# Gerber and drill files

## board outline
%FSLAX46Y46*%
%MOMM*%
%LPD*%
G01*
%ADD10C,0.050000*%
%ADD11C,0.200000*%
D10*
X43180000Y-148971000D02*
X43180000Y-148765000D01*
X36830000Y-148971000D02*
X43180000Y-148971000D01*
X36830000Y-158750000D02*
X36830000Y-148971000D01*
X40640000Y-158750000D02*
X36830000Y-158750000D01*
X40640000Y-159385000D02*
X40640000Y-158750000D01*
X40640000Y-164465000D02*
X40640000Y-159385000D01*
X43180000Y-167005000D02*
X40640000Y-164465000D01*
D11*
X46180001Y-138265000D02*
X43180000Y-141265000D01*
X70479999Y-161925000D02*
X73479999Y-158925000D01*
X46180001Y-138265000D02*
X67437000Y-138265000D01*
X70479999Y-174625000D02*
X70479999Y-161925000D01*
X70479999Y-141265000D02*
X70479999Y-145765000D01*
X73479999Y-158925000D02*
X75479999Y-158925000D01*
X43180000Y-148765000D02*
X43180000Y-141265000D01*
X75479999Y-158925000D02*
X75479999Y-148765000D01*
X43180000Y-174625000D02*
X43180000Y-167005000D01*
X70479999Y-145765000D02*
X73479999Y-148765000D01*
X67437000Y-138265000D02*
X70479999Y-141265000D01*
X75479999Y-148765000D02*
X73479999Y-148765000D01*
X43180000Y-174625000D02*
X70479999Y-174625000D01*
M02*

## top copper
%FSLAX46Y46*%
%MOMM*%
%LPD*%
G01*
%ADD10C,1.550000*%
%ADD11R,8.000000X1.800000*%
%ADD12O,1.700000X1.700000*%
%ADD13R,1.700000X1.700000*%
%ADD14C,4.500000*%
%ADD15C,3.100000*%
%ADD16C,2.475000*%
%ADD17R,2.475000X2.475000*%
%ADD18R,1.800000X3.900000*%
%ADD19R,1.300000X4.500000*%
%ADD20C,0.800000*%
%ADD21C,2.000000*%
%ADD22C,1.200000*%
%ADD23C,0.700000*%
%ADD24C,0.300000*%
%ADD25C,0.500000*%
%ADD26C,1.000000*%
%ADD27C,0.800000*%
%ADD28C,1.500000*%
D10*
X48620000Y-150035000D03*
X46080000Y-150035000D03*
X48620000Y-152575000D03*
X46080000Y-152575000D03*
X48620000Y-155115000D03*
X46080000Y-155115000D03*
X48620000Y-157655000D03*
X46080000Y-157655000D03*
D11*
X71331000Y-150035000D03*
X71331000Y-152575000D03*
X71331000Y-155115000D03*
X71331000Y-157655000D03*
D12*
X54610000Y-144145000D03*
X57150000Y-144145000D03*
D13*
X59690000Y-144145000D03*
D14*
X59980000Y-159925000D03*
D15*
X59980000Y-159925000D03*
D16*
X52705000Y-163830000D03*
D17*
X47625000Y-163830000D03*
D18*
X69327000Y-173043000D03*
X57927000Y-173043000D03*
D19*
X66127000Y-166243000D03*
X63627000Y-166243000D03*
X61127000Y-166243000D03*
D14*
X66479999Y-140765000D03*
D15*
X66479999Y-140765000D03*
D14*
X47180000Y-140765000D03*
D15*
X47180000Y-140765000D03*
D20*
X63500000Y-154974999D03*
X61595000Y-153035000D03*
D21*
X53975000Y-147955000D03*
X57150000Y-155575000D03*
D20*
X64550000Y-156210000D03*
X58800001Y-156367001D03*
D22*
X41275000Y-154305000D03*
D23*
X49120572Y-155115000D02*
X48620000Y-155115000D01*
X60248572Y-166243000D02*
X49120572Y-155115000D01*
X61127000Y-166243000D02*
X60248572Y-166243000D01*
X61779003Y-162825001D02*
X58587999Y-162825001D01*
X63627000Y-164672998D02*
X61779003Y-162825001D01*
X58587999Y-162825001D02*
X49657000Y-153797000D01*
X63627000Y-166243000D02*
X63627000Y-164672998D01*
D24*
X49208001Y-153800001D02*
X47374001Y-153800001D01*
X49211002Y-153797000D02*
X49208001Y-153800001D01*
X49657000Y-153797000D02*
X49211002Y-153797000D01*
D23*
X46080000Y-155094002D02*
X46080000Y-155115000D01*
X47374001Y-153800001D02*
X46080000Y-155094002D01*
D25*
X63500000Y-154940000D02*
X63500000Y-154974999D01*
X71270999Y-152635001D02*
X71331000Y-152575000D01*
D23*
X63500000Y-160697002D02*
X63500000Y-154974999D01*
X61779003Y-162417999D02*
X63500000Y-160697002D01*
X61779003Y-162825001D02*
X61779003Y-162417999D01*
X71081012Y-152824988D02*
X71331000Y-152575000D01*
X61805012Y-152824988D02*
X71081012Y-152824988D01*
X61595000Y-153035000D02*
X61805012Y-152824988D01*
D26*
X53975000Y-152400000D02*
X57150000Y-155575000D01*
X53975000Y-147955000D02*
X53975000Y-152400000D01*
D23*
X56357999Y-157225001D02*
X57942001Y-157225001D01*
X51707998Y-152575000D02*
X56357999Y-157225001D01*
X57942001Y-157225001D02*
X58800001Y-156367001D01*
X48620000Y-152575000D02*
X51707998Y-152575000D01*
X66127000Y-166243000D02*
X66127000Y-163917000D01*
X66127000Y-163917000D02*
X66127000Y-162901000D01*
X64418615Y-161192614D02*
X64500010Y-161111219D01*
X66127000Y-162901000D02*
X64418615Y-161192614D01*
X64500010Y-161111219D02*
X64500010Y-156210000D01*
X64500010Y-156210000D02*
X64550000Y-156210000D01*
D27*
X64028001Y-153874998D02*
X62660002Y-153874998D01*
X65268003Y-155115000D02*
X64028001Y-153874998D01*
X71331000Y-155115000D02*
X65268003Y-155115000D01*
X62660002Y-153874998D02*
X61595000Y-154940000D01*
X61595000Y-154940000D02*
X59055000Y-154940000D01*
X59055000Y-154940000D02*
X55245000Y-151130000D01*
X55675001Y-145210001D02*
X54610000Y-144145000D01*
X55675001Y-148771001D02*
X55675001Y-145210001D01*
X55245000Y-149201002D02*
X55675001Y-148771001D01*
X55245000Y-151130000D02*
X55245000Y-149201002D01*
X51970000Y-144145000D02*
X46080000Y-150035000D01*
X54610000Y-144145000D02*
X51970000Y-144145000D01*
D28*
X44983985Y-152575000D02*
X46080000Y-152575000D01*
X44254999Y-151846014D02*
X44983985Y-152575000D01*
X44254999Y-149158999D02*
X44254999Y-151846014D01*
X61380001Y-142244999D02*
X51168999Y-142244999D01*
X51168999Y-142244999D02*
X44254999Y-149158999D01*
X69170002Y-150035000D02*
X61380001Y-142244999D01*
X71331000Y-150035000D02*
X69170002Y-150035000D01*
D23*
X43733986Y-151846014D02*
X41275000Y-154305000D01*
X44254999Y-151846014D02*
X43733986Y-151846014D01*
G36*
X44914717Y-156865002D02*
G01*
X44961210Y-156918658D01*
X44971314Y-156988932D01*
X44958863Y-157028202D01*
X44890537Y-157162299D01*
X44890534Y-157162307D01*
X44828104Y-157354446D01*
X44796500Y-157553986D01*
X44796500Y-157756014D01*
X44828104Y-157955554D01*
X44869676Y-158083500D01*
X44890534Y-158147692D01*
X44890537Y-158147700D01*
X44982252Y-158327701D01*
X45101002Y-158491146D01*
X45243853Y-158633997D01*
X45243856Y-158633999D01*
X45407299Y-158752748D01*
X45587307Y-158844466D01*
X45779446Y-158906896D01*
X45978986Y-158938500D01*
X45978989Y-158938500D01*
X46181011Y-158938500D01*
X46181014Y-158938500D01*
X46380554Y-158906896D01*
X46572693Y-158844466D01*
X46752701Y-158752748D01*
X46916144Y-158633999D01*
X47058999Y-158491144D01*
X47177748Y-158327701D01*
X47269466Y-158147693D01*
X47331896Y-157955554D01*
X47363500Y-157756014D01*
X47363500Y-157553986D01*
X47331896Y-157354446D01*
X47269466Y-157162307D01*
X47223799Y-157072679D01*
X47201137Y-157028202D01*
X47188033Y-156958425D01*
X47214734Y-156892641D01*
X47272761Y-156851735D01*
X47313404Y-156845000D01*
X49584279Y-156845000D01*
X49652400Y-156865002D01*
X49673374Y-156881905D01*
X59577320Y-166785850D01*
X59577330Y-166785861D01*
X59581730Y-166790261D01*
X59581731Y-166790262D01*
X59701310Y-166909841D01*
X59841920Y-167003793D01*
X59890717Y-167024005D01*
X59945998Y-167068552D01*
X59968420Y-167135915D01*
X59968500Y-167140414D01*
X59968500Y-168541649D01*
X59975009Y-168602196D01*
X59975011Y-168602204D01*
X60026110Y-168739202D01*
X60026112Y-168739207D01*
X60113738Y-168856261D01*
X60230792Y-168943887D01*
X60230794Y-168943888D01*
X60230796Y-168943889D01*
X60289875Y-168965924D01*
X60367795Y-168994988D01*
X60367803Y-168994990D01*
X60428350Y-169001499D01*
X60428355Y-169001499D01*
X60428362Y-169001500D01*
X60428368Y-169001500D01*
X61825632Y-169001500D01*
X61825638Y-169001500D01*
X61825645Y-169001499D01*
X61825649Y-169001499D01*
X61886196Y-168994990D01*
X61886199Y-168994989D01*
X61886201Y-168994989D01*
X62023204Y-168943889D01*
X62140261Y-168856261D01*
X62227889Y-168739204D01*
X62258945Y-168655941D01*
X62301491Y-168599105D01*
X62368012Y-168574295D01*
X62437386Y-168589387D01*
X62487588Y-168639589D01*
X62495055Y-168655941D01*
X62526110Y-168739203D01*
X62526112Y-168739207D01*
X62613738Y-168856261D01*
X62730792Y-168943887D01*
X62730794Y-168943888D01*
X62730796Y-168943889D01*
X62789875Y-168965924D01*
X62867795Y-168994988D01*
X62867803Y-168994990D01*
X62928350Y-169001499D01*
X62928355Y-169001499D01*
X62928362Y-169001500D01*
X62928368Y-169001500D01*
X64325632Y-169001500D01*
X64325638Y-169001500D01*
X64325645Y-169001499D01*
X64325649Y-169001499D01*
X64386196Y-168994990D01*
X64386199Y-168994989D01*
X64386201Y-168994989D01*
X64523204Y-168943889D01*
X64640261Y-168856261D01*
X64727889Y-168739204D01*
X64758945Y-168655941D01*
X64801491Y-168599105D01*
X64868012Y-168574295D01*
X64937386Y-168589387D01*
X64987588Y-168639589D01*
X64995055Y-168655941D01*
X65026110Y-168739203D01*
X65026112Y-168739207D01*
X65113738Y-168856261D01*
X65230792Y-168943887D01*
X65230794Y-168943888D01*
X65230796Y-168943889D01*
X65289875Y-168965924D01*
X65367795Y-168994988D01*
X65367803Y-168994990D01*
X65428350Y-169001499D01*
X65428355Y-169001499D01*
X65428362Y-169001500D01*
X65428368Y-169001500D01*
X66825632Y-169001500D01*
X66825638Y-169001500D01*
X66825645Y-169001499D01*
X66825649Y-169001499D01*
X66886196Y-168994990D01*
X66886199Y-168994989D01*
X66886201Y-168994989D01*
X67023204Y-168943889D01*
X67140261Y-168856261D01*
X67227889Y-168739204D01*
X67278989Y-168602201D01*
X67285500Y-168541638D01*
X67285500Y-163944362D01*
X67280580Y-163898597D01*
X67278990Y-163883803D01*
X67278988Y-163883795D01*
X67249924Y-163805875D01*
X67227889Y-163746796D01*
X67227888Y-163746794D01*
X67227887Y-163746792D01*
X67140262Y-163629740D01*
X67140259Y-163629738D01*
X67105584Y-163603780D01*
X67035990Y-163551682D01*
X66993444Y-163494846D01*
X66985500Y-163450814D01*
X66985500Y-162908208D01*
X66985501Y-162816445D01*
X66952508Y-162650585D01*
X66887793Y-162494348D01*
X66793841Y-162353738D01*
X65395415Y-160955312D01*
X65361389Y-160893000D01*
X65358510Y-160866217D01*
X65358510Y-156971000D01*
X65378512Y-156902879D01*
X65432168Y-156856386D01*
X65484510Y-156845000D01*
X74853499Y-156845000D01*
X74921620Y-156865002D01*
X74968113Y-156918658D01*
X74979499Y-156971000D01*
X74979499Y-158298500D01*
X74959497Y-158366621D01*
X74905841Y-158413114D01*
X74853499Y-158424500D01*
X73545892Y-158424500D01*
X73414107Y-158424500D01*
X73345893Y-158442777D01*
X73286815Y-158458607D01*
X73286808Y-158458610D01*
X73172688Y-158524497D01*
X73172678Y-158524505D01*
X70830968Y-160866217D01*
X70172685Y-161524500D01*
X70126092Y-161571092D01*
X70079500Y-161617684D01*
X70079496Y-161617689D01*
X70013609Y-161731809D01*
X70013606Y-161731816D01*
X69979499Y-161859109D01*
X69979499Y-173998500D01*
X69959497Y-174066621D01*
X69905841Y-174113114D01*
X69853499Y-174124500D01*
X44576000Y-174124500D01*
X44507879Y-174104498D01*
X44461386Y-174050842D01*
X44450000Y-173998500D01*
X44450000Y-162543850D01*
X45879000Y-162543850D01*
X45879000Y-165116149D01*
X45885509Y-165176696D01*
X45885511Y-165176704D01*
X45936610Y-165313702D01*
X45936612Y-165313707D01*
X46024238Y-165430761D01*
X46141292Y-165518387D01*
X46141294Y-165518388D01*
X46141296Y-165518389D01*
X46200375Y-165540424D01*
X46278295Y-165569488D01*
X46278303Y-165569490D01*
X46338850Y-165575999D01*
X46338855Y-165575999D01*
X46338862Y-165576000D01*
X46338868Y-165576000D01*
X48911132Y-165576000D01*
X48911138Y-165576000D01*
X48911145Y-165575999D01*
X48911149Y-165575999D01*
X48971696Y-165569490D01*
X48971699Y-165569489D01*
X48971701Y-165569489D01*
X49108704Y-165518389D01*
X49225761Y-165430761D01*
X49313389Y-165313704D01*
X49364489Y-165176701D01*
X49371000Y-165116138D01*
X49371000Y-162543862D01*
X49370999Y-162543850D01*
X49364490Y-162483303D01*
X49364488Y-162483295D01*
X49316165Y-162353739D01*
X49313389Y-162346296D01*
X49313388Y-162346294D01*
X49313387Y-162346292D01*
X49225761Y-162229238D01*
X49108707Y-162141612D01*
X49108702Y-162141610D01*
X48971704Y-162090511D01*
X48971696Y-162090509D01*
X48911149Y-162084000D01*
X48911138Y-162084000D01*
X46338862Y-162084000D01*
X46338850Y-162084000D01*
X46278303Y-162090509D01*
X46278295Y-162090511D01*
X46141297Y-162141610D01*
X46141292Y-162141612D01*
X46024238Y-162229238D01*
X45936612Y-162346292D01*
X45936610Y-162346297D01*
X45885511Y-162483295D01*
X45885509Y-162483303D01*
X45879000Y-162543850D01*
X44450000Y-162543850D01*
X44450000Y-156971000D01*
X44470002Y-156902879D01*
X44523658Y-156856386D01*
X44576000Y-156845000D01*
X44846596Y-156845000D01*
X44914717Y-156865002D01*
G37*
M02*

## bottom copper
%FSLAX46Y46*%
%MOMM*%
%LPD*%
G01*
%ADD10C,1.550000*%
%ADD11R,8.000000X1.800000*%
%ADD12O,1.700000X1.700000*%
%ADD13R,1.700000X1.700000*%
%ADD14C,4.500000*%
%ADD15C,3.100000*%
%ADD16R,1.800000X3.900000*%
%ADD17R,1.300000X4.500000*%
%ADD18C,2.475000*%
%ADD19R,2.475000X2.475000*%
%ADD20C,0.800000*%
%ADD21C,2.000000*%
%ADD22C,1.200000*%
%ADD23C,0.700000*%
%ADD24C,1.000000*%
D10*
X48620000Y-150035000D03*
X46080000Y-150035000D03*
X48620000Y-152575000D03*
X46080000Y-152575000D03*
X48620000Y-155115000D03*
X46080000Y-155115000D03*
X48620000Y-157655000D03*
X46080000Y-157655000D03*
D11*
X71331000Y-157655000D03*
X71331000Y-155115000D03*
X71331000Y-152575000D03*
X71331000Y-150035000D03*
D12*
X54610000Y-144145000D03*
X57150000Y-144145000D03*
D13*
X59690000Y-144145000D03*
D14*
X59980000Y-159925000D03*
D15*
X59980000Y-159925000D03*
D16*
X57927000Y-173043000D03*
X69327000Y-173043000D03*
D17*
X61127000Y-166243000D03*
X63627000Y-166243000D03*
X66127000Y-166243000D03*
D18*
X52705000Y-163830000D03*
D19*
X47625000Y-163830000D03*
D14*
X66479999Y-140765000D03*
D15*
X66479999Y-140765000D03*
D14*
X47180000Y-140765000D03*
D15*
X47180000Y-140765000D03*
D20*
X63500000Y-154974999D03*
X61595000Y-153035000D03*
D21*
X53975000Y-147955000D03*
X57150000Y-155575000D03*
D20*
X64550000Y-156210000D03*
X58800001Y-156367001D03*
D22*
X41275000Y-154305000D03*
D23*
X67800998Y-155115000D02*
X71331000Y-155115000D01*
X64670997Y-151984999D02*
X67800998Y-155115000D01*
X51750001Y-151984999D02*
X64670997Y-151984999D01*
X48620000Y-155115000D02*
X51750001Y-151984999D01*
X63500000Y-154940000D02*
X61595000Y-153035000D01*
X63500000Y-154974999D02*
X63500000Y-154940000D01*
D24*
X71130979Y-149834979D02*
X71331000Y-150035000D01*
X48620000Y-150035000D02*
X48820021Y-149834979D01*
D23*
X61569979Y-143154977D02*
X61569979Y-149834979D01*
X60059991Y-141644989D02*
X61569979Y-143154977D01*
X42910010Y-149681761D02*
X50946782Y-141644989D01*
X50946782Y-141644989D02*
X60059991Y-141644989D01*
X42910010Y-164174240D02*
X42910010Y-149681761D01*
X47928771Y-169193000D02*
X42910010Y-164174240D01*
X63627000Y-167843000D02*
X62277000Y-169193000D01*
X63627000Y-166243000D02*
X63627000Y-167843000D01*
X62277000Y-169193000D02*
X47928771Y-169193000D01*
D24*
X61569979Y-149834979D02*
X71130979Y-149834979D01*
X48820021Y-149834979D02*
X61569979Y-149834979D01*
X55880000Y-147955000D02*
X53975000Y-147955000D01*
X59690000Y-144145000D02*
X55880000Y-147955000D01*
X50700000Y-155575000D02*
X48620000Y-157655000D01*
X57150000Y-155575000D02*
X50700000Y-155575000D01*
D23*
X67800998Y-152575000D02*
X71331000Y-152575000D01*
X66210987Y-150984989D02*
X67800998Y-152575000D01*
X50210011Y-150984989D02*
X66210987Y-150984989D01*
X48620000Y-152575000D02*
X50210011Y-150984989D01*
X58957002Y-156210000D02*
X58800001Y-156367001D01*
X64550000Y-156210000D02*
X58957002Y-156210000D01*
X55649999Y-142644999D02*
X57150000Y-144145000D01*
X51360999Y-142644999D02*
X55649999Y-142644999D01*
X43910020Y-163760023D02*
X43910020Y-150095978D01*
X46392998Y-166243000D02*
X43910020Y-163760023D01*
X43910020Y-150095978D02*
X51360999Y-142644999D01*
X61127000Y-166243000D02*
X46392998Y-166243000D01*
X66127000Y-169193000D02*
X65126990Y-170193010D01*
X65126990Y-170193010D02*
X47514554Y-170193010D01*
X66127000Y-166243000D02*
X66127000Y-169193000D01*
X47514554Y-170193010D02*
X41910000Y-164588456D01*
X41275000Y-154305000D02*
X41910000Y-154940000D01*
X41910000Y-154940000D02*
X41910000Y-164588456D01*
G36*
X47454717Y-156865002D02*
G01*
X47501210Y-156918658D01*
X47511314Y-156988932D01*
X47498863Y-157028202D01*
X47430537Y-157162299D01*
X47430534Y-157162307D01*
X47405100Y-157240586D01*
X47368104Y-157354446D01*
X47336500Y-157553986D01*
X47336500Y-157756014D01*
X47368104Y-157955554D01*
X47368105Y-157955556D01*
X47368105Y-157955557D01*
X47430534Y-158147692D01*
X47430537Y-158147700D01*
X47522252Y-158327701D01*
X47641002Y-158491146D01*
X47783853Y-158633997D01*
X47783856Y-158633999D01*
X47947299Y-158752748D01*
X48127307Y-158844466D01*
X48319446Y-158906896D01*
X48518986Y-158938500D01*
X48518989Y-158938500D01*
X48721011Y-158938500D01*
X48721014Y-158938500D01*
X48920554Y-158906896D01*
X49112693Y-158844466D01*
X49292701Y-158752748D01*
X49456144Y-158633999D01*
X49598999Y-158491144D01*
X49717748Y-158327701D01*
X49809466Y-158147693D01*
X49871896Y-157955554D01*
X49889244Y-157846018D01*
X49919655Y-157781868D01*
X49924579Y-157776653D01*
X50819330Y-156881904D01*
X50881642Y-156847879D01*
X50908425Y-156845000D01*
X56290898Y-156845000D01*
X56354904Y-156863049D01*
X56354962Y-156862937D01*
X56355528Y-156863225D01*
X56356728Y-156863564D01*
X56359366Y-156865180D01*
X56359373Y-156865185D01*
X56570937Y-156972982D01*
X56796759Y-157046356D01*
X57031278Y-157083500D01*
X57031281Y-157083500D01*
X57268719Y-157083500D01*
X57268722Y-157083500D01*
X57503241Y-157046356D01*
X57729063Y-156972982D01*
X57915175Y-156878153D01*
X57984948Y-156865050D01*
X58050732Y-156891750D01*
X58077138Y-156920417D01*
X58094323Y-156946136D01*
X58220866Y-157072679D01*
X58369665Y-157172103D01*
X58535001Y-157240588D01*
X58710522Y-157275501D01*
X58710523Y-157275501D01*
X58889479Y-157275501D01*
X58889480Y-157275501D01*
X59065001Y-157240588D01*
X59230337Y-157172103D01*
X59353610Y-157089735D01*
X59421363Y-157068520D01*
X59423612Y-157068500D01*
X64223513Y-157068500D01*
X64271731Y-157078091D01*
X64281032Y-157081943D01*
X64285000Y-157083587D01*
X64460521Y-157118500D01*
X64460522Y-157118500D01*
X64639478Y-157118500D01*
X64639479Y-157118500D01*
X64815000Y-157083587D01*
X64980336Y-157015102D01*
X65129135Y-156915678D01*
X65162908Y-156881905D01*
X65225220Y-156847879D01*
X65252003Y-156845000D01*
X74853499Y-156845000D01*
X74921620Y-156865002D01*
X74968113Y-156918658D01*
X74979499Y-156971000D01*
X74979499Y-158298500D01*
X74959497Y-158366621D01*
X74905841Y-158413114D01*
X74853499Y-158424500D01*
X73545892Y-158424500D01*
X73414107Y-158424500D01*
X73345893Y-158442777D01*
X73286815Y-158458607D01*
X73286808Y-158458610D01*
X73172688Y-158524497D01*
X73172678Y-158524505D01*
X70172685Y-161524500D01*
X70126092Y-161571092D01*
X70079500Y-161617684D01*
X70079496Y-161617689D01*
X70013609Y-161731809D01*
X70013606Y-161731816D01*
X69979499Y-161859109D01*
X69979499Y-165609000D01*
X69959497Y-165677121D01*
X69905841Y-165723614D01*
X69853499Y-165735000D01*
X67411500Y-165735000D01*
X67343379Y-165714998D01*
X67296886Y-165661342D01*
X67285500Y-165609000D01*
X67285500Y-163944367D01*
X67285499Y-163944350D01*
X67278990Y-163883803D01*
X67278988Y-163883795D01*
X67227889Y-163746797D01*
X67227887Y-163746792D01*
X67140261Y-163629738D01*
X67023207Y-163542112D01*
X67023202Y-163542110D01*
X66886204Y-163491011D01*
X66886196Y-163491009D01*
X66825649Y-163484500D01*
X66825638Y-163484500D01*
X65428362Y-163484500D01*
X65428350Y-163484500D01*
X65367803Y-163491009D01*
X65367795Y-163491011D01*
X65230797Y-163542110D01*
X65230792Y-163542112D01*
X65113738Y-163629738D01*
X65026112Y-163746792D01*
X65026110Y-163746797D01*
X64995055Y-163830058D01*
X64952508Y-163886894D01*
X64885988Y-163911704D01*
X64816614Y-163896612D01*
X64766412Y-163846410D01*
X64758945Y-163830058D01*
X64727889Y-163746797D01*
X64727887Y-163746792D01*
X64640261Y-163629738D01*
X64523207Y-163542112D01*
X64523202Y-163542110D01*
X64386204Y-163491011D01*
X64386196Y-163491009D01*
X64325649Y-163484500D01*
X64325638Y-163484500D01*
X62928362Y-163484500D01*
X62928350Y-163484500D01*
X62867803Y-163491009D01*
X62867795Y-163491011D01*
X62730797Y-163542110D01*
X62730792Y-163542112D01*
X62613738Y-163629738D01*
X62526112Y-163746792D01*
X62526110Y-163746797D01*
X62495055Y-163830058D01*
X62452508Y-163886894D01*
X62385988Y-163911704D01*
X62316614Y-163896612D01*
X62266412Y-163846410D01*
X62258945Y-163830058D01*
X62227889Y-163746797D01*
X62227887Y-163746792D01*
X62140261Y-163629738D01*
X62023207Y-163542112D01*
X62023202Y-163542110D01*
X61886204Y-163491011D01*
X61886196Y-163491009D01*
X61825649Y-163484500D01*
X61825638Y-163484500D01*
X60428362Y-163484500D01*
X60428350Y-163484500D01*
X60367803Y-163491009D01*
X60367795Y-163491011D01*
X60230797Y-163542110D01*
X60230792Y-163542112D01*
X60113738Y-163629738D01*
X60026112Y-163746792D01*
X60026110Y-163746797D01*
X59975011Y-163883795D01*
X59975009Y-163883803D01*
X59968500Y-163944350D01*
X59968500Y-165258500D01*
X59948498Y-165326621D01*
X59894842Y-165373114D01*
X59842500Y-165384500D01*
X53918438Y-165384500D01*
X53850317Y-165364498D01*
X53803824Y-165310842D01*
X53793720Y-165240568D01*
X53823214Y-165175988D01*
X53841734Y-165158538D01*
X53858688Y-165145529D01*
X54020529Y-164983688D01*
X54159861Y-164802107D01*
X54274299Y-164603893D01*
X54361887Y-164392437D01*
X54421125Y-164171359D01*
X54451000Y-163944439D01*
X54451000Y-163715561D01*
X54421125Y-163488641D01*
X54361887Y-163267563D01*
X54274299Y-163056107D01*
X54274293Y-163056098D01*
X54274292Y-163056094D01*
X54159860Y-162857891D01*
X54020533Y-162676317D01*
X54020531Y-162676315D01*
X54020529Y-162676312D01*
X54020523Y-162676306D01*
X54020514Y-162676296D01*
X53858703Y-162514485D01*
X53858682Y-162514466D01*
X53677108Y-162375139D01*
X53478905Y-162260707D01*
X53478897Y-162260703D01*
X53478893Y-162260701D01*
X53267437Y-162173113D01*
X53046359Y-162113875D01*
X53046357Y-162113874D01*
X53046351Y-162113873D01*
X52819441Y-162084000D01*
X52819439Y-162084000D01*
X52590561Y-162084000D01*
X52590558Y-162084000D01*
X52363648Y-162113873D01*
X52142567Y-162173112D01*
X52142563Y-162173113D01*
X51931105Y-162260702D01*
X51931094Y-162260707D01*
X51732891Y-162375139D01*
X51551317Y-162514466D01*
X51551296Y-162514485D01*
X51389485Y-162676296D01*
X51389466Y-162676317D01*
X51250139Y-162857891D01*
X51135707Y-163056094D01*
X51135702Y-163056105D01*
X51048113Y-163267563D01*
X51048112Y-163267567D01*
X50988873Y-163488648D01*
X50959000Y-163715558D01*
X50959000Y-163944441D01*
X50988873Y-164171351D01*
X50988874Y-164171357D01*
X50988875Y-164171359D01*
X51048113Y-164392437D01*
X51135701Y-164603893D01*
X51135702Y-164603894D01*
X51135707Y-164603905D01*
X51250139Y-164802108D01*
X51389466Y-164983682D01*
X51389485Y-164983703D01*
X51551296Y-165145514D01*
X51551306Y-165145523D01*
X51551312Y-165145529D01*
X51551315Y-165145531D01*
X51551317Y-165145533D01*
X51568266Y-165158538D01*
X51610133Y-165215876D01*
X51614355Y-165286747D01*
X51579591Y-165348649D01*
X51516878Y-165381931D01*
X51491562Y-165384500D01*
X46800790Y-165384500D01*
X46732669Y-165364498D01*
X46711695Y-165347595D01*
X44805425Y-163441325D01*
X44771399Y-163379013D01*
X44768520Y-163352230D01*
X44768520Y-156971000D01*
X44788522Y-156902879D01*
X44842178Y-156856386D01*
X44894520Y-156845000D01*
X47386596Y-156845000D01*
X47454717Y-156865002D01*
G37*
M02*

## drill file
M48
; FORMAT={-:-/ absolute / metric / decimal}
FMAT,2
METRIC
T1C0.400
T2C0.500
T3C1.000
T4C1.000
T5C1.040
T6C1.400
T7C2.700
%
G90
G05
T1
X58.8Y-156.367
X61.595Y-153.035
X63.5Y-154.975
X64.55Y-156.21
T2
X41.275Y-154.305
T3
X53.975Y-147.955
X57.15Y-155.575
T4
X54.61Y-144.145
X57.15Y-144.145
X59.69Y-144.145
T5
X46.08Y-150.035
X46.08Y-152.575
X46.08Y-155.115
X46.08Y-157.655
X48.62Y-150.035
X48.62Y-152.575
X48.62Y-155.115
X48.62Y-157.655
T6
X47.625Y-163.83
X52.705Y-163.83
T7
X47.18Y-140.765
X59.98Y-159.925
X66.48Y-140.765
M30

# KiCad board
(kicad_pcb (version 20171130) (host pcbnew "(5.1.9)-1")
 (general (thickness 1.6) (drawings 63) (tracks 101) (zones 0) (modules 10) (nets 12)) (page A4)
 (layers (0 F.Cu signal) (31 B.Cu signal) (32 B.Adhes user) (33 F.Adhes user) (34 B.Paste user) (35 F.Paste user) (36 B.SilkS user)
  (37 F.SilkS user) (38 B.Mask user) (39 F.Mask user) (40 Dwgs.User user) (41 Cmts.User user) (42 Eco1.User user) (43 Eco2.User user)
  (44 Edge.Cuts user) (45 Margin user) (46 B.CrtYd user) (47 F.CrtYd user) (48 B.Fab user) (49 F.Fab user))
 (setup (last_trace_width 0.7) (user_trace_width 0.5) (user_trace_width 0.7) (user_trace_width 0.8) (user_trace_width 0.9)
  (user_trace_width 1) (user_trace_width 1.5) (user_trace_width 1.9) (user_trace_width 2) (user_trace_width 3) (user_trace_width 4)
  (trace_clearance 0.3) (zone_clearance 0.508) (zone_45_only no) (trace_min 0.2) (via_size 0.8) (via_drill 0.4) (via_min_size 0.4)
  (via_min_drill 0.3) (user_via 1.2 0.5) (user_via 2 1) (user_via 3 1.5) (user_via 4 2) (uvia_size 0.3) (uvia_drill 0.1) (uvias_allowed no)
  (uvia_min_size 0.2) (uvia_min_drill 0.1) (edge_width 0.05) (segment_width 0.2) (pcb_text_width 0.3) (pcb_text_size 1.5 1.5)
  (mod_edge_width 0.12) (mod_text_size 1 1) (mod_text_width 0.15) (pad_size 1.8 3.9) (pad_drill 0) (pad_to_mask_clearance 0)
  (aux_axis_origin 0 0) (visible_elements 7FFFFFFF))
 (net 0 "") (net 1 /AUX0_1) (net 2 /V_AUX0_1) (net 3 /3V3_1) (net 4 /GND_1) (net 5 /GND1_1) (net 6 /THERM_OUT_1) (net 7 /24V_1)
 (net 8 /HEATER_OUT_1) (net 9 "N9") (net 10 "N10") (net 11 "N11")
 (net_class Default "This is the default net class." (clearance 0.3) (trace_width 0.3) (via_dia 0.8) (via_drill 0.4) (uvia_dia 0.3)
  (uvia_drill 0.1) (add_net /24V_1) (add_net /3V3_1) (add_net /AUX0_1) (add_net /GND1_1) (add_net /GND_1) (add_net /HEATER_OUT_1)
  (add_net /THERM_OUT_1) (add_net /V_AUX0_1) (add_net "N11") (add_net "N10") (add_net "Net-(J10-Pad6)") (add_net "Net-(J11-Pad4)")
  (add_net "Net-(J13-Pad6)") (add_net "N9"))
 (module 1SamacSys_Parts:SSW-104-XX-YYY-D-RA (layer F.Cu) (at 46.08 157.655 270)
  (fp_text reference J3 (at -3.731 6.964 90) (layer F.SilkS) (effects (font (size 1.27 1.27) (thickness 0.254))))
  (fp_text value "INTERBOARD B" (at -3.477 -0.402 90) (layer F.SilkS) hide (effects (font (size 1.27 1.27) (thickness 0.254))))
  (pad 8 thru_hole circle (at -7.62 -2.54 270) (size 1.55 1.55) (drill 1.04) (layers *.Cu *.Mask) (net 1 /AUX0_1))
  (pad 7 thru_hole circle (at -7.62 0 270) (size 1.55 1.55) (drill 1.04) (layers *.Cu *.Mask) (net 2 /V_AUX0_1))
  (pad 6 thru_hole circle (at -5.08 -2.54 270) (size 1.55 1.55) (drill 1.04) (layers *.Cu *.Mask) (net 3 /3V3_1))
  (pad 5 thru_hole circle (at -5.08 0 270) (size 1.55 1.55) (drill 1.04) (layers *.Cu *.Mask) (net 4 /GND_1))
  (pad 4 thru_hole circle (at -2.54 -2.54 270) (size 1.55 1.55) (drill 1.04) (layers *.Cu *.Mask) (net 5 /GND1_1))
  (pad 3 thru_hole circle (at -2.54 0 270) (size 1.55 1.55) (drill 1.04) (layers *.Cu *.Mask) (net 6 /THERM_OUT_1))
  (pad 2 thru_hole circle (at 0 -2.54 270) (size 1.55 1.55) (drill 1.04) (layers *.Cu *.Mask) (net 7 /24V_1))
  (pad 1 thru_hole circle (at 0 0 270) (size 1.55 1.55) (drill 1.04) (layers *.Cu *.Mask) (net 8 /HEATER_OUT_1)))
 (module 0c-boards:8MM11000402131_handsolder (layer F.Cu) (at 71.87 153.845 270)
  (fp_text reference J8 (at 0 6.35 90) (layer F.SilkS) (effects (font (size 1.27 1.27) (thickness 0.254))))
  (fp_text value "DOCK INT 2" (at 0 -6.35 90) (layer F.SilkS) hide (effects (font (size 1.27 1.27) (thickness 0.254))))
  (pad 1 smd rect (at -3.81 0.539 270) (size 1.8 8) (layers F.Cu F.Paste F.Mask) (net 4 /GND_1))
  (pad 2 smd rect (at -1.27 0.539 270) (size 1.8 8) (layers F.Cu F.Paste F.Mask) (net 6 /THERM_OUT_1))
  (pad 3 smd rect (at 1.27 0.539 270) (size 1.8 8) (layers F.Cu F.Paste F.Mask) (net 2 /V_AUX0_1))
  (pad 4 smd rect (at 3.81 0.539 270) (size 1.8 8) (layers F.Cu F.Paste F.Mask) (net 7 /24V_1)))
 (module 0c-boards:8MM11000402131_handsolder (layer B.Cu) (at 71.87 153.845 90)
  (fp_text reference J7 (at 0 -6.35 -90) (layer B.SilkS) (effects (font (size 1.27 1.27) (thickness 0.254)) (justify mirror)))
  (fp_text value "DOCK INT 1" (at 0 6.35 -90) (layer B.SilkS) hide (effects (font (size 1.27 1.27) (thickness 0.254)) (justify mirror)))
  (pad 1 smd rect (at -3.81 -0.539 90) (size 1.8 8) (layers B.Cu B.Paste B.Mask) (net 8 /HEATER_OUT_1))
  (pad 2 smd rect (at -1.27 -0.539 90) (size 1.8 8) (layers B.Cu B.Paste B.Mask) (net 5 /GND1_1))
  (pad 3 smd rect (at 1.27 -0.539 90) (size 1.8 8) (layers B.Cu B.Paste B.Mask) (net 3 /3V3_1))
  (pad 4 smd rect (at 3.81 -0.539 90) (size 1.8 8) (layers B.Cu B.Paste B.Mask) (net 1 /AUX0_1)))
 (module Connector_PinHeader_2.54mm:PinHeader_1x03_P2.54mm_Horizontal (layer B.Cu) (at 59.69 144.145 90)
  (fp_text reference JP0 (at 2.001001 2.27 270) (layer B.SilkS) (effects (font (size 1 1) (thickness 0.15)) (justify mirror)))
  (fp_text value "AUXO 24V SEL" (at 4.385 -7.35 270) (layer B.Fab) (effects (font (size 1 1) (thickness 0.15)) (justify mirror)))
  (pad 3 thru_hole oval (at 0 -5.08 90) (size 1.7 1.7) (drill 1) (layers *.Cu *.Mask) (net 2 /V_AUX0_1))
  (pad 2 thru_hole oval (at 0 -2.54 90) (size 1.7 1.7) (drill 1) (layers *.Cu *.Mask) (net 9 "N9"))
  (pad 1 thru_hole rect (at 0 0 90) (size 1.7 1.7) (drill 1) (layers *.Cu *.Mask) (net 7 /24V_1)))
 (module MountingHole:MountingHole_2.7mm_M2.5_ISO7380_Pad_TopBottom (layer F.Cu) (at 59.98 159.925)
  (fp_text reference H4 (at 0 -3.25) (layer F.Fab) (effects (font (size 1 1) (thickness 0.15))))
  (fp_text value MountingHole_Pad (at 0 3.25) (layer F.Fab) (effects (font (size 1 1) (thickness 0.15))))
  (pad 1 connect circle (at 0 0) (size 4.5 4.5) (layers B.Cu B.Mask) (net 8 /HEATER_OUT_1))
  (pad 1 connect circle (at 0 0) (size 4.5 4.5) (layers F.Cu F.Mask) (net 8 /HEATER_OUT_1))
  (pad 1 thru_hole circle (at 0 0) (size 3.1 3.1) (drill 2.7) (layers *.Cu *.Mask) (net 8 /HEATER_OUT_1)))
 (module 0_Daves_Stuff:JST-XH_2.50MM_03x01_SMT (layer B.Cu) (at 63.627 166.243 180)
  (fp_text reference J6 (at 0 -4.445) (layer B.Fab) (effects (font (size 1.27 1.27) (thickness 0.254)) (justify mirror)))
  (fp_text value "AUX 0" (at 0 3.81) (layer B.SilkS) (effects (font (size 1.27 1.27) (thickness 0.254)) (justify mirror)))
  (pad 5 smd rect (at 5.7 -6.8 180) (size 1.8 3.9) (layers B.Cu B.Paste B.Mask))
  (pad 4 smd rect (at -5.7 -6.8 180) (size 1.8 3.9) (layers B.Cu B.Paste B.Mask))
  (pad 3 smd rect (at 2.5 0 180) (size 1.3 4.5) (layers B.Cu B.Paste B.Mask) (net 9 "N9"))
  (pad 2 smd rect (at 0 0 180) (size 1.3 4.5) (layers B.Cu B.Paste B.Mask) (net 1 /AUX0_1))
  (pad 1 smd rect (at -2.5 0 180) (size 1.3 4.5) (layers B.Cu B.Paste B.Mask) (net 4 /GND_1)))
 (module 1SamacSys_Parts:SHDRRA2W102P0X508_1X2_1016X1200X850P (layer F.Cu) (at 47.625 163.83 180)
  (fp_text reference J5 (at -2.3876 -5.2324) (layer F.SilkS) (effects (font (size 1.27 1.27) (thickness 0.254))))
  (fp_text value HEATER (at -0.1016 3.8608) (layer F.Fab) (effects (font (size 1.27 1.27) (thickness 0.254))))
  (pad 2 thru_hole circle (at -5.08 0 180) (size 2.475 2.475) (drill 1.4) (layers *.Cu *.Mask) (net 7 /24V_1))
  (pad 1 thru_hole rect (at 0 0 180) (size 2.475 2.475) (drill 1.4) (layers *.Cu *.Mask) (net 8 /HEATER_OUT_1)))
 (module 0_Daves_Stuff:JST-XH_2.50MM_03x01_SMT (layer F.Cu) (at 63.627 166.243)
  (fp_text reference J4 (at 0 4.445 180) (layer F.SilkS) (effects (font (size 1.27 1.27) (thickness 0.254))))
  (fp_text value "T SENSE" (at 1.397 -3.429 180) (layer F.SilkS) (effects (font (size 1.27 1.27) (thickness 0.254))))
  (pad 5 smd rect (at 5.7 6.8) (size 1.8 3.9) (layers F.Cu F.Paste F.Mask) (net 7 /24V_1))
  (pad 4 smd rect (at -5.7 6.8) (size 1.8 3.9) (layers F.Cu F.Paste F.Mask) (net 7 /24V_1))
  (pad 3 smd rect (at 2.5 0) (size 1.3 4.5) (layers F.Cu F.Paste F.Mask) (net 3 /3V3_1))
  (pad 2 smd rect (at 0 0) (size 1.3 4.5) (layers F.Cu F.Paste F.Mask) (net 6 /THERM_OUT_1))
  (pad 1 smd rect (at -2.5 0) (size 1.3 4.5) (layers F.Cu F.Paste F.Mask) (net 5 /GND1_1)))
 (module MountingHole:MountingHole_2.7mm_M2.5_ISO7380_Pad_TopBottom (layer F.Cu) (at 66.479999 140.765)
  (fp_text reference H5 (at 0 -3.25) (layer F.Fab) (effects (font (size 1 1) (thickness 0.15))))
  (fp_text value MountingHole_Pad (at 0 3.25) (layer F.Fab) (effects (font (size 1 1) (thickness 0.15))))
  (pad 1 connect circle (at 0 0) (size 4.5 4.5) (layers B.Cu B.Mask) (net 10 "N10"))
  (pad 1 connect circle (at 0 0) (size 4.5 4.5) (layers F.Cu F.Mask) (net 10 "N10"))
  (pad 1 thru_hole circle (at 0 0) (size 3.1 3.1) (drill 2.7) (layers *.Cu *.Mask) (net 10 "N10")))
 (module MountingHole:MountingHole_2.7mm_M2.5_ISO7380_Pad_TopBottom (layer F.Cu) (at 47.18 140.765)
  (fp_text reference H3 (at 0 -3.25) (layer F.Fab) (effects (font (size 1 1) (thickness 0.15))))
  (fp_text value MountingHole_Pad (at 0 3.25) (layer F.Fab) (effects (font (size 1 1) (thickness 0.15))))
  (pad 1 connect circle (at 0 0) (size 4.5 4.5) (layers B.Cu B.Mask) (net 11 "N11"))
  (pad 1 connect circle (at 0 0) (size 4.5 4.5) (layers F.Cu F.Mask) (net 11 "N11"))
  (pad 1 thru_hole circle (at 0 0) (size 3.1 3.1) (drill 2.7) (layers *.Cu *.Mask) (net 11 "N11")))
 (gr_line (start 43.18 148.971) (end 43.18 148.765) (layer Edge.Cuts) (width 0.05))
 (gr_line (start 36.83 148.971) (end 43.18 148.971) (layer Edge.Cuts) (width 0.05))
 (gr_line (start 36.83 158.75) (end 36.83 148.971) (layer Edge.Cuts) (width 0.05))
 (gr_line (start 40.64 158.75) (end 36.83 158.75) (layer Edge.Cuts) (width 0.05))
 (gr_line (start 40.64 159.385) (end 40.64 158.75) (layer Edge.Cuts) (width 0.05))
 (gr_line (start 40.64 164.465) (end 40.64 159.385) (layer Edge.Cuts) (width 0.05))
 (gr_line (start 43.18 167.005) (end 40.64 164.465) (layer Edge.Cuts) (width 0.05))
 (gr_line (start 46.180001 138.265) (end 43.18 141.265) (layer Edge.Cuts) (width 0.2))
 (gr_line (start 70.479999 161.925) (end 73.479999 158.925) (layer Edge.Cuts) (width 0.2))
 (gr_line (start 46.180001 138.265) (end 67.437 138.265) (layer Edge.Cuts) (width 0.2))
 (gr_line (start 70.479999 174.625) (end 70.479999 161.925) (layer Edge.Cuts) (width 0.2))
 (gr_line (start 70.479999 141.265) (end 70.479999 145.765) (layer Edge.Cuts) (width 0.2))
 (gr_line (start 73.479999 158.925) (end 75.479999 158.925) (layer Edge.Cuts) (width 0.2))
 (gr_line (start 43.18 148.765) (end 43.18 141.265) (layer Edge.Cuts) (width 0.2))
 (gr_line (start 75.479999 158.925) (end 75.479999 148.765) (layer Edge.Cuts) (width 0.2))
 (gr_line (start 43.18 174.625) (end 43.18 167.005) (layer Edge.Cuts) (width 0.2))
 (gr_line (start 70.479999 145.765) (end 73.479999 148.765) (layer Edge.Cuts) (width 0.2))
 (gr_line (start 67.437 138.265) (end 70.479999 141.265) (layer Edge.Cuts) (width 0.2))
 (gr_line (start 75.479999 148.765) (end 73.479999 148.765) (layer Edge.Cuts) (width 0.2))
 (gr_line (start 43.18 174.625) (end 70.479999 174.625) (layer Edge.Cuts) (width 0.2))
 (segment (start 49.120572 155.115) (end 48.62 155.115) (width 0.7) (layer F.Cu) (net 5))
 (segment (start 60.248572 166.243) (end 49.120572 155.115) (width 0.7) (layer F.Cu) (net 5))
 (segment (start 61.127 166.243) (end 60.248572 166.243) (width 0.7) (layer F.Cu) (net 5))
 (segment (start 67.800998 155.115) (end 71.331 155.115) (width 0.7) (layer B.Cu) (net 5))
 (segment (start 64.670997 151.984999) (end 67.800998 155.115) (width 0.7) (layer B.Cu) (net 5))
 (segment (start 51.750001 151.984999) (end 64.670997 151.984999) (width 0.7) (layer B.Cu) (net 5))
 (segment (start 48.62 155.115) (end 51.750001 151.984999) (width 0.7) (layer B.Cu) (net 5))
 (segment (start 61.779003 162.825001) (end 58.587999 162.825001) (width 0.7) (layer F.Cu) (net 6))
 (segment (start 63.627 164.672998) (end 61.779003 162.825001) (width 0.7) (layer F.Cu) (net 6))
 (segment (start 58.587999 162.825001) (end 49.657 153.797) (width 0.7) (layer F.Cu) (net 6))
 (segment (start 63.627 166.243) (end 63.627 164.672998) (width 0.7) (layer F.Cu) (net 6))
 (segment (start 49.208001 153.800001) (end 47.374001 153.800001) (width 0.3) (layer F.Cu) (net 6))
 (segment (start 49.211002 153.797) (end 49.208001 153.800001) (width 0.3) (layer F.Cu) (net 6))
 (segment (start 49.657 153.797) (end 49.211002 153.797) (width 0.3) (layer F.Cu) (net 6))
 (segment (start 46.08 155.094002) (end 46.08 155.115) (width 0.7) (layer F.Cu) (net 6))
 (segment (start 47.374001 153.800001) (end 46.08 155.094002) (width 0.7) (layer F.Cu) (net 6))
 (segment (start 63.5 154.94) (end 63.5 154.974999) (width 0.5) (layer F.Cu) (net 6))
 (via (at 63.5 154.974999) (size 0.8) (drill 0.4) (layers F.Cu B.Cu) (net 6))
 (via (at 61.595 153.035) (size 0.8) (drill 0.4) (layers F.Cu B.Cu) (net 6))
 (segment (start 71.270999 152.635001) (end 71.331 152.575) (width 0.5) (layer F.Cu) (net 6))
 (segment (start 63.5 160.697002) (end 63.5 154.974999) (width 0.7) (layer F.Cu) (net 6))
 (segment (start 61.779003 162.417999) (end 63.5 160.697002) (width 0.7) (layer F.Cu) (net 6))
 (segment (start 61.779003 162.825001) (end 61.779003 162.417999) (width 0.7) (layer F.Cu) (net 6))
 (segment (start 63.5 154.94) (end 61.595 153.035) (width 0.7) (layer B.Cu) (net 6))
 (segment (start 63.5 154.974999) (end 63.5 154.94) (width 0.7) (layer B.Cu) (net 6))
 (segment (start 71.081012 152.824988) (end 71.331 152.575) (width 0.7) (layer F.Cu) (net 6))
 (segment (start 61.805012 152.824988) (end 71.081012 152.824988) (width 0.7) (layer F.Cu) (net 6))
 (segment (start 61.595 153.035) (end 61.805012 152.824988) (width 0.7) (layer F.Cu) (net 6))
 (segment (start 71.130979 149.834979) (end 71.331 150.035) (width 1) (layer B.Cu) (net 1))
 (segment (start 48.62 150.035) (end 48.820021 149.834979) (width 1) (layer B.Cu) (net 1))
 (segment (start 61.569979 143.154977) (end 61.569979 149.834979) (width 0.7) (layer B.Cu) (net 1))
 (segment (start 60.059991 141.644989) (end 61.569979 143.154977) (width 0.7) (layer B.Cu) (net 1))
 (segment (start 42.91001 149.681761) (end 50.946782 141.644989) (width 0.7) (layer B.Cu) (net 1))
 (segment (start 50.946782 141.644989) (end 60.059991 141.644989) (width 0.7) (layer B.Cu) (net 1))
 (segment (start 42.91001 164.17424) (end 42.91001 149.681761) (width 0.7) (layer B.Cu) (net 1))
 (segment (start 47.928771 169.193) (end 42.91001 164.17424) (width 0.7) (layer B.Cu) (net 1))
 (segment (start 63.627 167.843) (end 62.277 169.193) (width 0.7) (layer B.Cu) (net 1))
 (segment (start 63.627 166.243) (end 63.627 167.843) (width 0.7) (layer B.Cu) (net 1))
 (segment (start 62.277 169.193) (end 47.928771 169.193) (width 0.7) (layer B.Cu) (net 1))
 (segment (start 61.569979 149.834979) (end 71.130979 149.834979) (width 1) (layer B.Cu) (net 1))
 (segment (start 48.820021 149.834979) (end 61.569979 149.834979) (width 1) (layer B.Cu) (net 1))
 (via (at 53.975 147.955) (size 2) (drill 1) (layers F.Cu B.Cu) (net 7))
 (segment (start 55.88 147.955) (end 53.975 147.955) (width 1) (layer B.Cu) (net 7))
 (segment (start 59.69 144.145) (end 55.88 147.955) (width 1) (layer B.Cu) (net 7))
 (via (at 57.15 155.575) (size 2) (drill 1) (layers F.Cu B.Cu) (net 7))
 (segment (start 53.975 152.4) (end 57.15 155.575) (width 1) (layer F.Cu) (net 7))
 (segment (start 53.975 147.955) (end 53.975 152.4) (width 1) (layer F.Cu) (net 7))
 (segment (start 50.7 155.575) (end 48.62 157.655) (width 1) (layer B.Cu) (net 7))
 (segment (start 57.15 155.575) (end 50.7 155.575) (width 1) (layer B.Cu) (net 7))
 (segment (start 56.357999 157.225001) (end 57.942001 157.225001) (width 0.7) (layer F.Cu) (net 3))
 (segment (start 51.707998 152.575) (end 56.357999 157.225001) (width 0.7) (layer F.Cu) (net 3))
 (segment (start 57.942001 157.225001) (end 58.800001 156.367001) (width 0.7) (layer F.Cu) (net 3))
 (segment (start 48.62 152.575) (end 51.707998 152.575) (width 0.7) (layer F.Cu) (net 3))
 (segment (start 67.800998 152.575) (end 71.331 152.575) (width 0.7) (layer B.Cu) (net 3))
 (segment (start 66.210987 150.984989) (end 67.800998 152.575) (width 0.7) (layer B.Cu) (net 3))
 (segment (start 50.210011 150.984989) (end 66.210987 150.984989) (width 0.7) (layer B.Cu) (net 3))
 (segment (start 48.62 152.575) (end 50.210011 150.984989) (width 0.7) (layer B.Cu) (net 3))
 (segment (start 66.127 166.243) (end 66.127 163.917) (width 0.7) (layer F.Cu) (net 3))
 (segment (start 66.127 163.917) (end 66.127 162.901) (width 0.7) (layer F.Cu) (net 3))
 (segment (start 64.418615 161.192614) (end 64.50001 161.111219) (width 0.7) (layer F.Cu) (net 3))
 (segment (start 66.127 162.901) (end 64.418615 161.192614) (width 0.7) (layer F.Cu) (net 3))
 (segment (start 64.50001 161.111219) (end 64.50001 156.21) (width 0.7) (layer F.Cu) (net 3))
 (via (at 64.55 156.21) (size 0.8) (drill 0.4) (layers F.Cu B.Cu) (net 3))
 (segment (start 64.50001 156.21) (end 64.55 156.21) (width 0.7) (layer F.Cu) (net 3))
 (via (at 58.800001 156.367001) (size 0.8) (drill 0.4) (layers F.Cu B.Cu) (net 3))
 (segment (start 58.957002 156.21) (end 58.800001 156.367001) (width 0.7) (layer B.Cu) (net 3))
 (segment (start 64.55 156.21) (end 58.957002 156.21) (width 0.7) (layer B.Cu) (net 3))
 (segment (start 64.028001 153.874998) (end 62.660002 153.874998) (width 0.8) (layer F.Cu) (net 2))
 (segment (start 65.268003 155.115) (end 64.028001 153.874998) (width 0.8) (layer F.Cu) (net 2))
 (segment (start 71.331 155.115) (end 65.268003 155.115) (width 0.8) (layer F.Cu) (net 2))
 (segment (start 62.660002 153.874998) (end 61.595 154.94) (width 0.8) (layer F.Cu) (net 2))
 (segment (start 61.595 154.94) (end 59.055 154.94) (width 0.8) (layer F.Cu) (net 2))
 (segment (start 59.055 154.94) (end 55.245 151.13) (width 0.8) (layer F.Cu) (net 2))
 (segment (start 55.675001 145.210001) (end 54.61 144.145) (width 0.8) (layer F.Cu) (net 2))
 (segment (start 55.675001 148.771001) (end 55.675001 145.210001) (width 0.8) (layer F.Cu) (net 2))
 (segment (start 55.245 149.201002) (end 55.675001 148.771001) (width 0.8) (layer F.Cu) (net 2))
 (segment (start 55.245 151.13) (end 55.245 149.201002) (width 0.8) (layer F.Cu) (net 2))
 (segment (start 51.97 144.145) (end 46.08 150.035) (width 0.8) (layer F.Cu) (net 2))
 (segment (start 54.61 144.145) (end 51.97 144.145) (width 0.8) (layer F.Cu) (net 2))
 (segment (start 55.649999 142.644999) (end 57.15 144.145) (width 0.7) (layer B.Cu) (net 9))
 (segment (start 51.360999 142.644999) (end 55.649999 142.644999) (width 0.7) (layer B.Cu) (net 9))
 (segment (start 43.91002 163.760023) (end 43.91002 150.095978) (width 0.7) (layer B.Cu) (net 9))
 (segment (start 46.392998 166.243) (end 43.91002 163.760023) (width 0.7) (layer B.Cu) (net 9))
 (segment (start 43.91002 150.095978) (end 51.360999 142.644999) (width 0.7) (layer B.Cu) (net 9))
 (segment (start 61.127 166.243) (end 46.392998 166.243) (width 0.7) (layer B.Cu) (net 9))
 (segment (start 44.983985 152.575) (end 46.08 152.575) (width 1.5) (layer F.Cu) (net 4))
 (segment (start 44.254999 151.846014) (end 44.983985 152.575) (width 1.5) (layer F.Cu) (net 4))
 (segment (start 44.254999 149.158999) (end 44.254999 151.846014) (width 1.5) (layer F.Cu) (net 4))
 (segment (start 61.380001 142.244999) (end 51.168999 142.244999) (width 1.5) (layer F.Cu) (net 4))
 (segment (start 51.168999 142.244999) (end 44.254999 149.158999) (width 1.5) (layer F.Cu) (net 4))
 (segment (start 69.170002 150.035) (end 61.380001 142.244999) (width 1.5) (layer F.Cu) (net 4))
 (segment (start 71.331 150.035) (end 69.170002 150.035) (width 1.5) (layer F.Cu) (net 4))
 (segment (start 66.127 169.193) (end 65.12699 170.19301) (width 0.7) (layer B.Cu) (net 4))
 (segment (start 65.12699 170.19301) (end 47.514554 170.19301) (width 0.7) (layer B.Cu) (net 4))
 (segment (start 66.127 166.243) (end 66.127 169.193) (width 0.7) (layer B.Cu) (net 4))
 (segment (start 47.514554 170.19301) (end 41.91 164.588456) (width 0.7) (layer B.Cu) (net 4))
 (segment (start 43.733986 151.846014) (end 41.275 154.305) (width 0.7) (layer F.Cu) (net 4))
 (segment (start 44.254999 151.846014) (end 43.733986 151.846014) (width 0.7) (layer F.Cu) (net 4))
 (via (at 41.275 154.305) (size 1.2) (drill 0.5) (layers F.Cu B.Cu) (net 4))
 (segment (start 41.275 154.305) (end 41.91 154.94) (width 0.7) (layer B.Cu) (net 4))
 (segment (start 41.91 154.94) (end 41.91 164.588456) (width 0.7) (layer B.Cu) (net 4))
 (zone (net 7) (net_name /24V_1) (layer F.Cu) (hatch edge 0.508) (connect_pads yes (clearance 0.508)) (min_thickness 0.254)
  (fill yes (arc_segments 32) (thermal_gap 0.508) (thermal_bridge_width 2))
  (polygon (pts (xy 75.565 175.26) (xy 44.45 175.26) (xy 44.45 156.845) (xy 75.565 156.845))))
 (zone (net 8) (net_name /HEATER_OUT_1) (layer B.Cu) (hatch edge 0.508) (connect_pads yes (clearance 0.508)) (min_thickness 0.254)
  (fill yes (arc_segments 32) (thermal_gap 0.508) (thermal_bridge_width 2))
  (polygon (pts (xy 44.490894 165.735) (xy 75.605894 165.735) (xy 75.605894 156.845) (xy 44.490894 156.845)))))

